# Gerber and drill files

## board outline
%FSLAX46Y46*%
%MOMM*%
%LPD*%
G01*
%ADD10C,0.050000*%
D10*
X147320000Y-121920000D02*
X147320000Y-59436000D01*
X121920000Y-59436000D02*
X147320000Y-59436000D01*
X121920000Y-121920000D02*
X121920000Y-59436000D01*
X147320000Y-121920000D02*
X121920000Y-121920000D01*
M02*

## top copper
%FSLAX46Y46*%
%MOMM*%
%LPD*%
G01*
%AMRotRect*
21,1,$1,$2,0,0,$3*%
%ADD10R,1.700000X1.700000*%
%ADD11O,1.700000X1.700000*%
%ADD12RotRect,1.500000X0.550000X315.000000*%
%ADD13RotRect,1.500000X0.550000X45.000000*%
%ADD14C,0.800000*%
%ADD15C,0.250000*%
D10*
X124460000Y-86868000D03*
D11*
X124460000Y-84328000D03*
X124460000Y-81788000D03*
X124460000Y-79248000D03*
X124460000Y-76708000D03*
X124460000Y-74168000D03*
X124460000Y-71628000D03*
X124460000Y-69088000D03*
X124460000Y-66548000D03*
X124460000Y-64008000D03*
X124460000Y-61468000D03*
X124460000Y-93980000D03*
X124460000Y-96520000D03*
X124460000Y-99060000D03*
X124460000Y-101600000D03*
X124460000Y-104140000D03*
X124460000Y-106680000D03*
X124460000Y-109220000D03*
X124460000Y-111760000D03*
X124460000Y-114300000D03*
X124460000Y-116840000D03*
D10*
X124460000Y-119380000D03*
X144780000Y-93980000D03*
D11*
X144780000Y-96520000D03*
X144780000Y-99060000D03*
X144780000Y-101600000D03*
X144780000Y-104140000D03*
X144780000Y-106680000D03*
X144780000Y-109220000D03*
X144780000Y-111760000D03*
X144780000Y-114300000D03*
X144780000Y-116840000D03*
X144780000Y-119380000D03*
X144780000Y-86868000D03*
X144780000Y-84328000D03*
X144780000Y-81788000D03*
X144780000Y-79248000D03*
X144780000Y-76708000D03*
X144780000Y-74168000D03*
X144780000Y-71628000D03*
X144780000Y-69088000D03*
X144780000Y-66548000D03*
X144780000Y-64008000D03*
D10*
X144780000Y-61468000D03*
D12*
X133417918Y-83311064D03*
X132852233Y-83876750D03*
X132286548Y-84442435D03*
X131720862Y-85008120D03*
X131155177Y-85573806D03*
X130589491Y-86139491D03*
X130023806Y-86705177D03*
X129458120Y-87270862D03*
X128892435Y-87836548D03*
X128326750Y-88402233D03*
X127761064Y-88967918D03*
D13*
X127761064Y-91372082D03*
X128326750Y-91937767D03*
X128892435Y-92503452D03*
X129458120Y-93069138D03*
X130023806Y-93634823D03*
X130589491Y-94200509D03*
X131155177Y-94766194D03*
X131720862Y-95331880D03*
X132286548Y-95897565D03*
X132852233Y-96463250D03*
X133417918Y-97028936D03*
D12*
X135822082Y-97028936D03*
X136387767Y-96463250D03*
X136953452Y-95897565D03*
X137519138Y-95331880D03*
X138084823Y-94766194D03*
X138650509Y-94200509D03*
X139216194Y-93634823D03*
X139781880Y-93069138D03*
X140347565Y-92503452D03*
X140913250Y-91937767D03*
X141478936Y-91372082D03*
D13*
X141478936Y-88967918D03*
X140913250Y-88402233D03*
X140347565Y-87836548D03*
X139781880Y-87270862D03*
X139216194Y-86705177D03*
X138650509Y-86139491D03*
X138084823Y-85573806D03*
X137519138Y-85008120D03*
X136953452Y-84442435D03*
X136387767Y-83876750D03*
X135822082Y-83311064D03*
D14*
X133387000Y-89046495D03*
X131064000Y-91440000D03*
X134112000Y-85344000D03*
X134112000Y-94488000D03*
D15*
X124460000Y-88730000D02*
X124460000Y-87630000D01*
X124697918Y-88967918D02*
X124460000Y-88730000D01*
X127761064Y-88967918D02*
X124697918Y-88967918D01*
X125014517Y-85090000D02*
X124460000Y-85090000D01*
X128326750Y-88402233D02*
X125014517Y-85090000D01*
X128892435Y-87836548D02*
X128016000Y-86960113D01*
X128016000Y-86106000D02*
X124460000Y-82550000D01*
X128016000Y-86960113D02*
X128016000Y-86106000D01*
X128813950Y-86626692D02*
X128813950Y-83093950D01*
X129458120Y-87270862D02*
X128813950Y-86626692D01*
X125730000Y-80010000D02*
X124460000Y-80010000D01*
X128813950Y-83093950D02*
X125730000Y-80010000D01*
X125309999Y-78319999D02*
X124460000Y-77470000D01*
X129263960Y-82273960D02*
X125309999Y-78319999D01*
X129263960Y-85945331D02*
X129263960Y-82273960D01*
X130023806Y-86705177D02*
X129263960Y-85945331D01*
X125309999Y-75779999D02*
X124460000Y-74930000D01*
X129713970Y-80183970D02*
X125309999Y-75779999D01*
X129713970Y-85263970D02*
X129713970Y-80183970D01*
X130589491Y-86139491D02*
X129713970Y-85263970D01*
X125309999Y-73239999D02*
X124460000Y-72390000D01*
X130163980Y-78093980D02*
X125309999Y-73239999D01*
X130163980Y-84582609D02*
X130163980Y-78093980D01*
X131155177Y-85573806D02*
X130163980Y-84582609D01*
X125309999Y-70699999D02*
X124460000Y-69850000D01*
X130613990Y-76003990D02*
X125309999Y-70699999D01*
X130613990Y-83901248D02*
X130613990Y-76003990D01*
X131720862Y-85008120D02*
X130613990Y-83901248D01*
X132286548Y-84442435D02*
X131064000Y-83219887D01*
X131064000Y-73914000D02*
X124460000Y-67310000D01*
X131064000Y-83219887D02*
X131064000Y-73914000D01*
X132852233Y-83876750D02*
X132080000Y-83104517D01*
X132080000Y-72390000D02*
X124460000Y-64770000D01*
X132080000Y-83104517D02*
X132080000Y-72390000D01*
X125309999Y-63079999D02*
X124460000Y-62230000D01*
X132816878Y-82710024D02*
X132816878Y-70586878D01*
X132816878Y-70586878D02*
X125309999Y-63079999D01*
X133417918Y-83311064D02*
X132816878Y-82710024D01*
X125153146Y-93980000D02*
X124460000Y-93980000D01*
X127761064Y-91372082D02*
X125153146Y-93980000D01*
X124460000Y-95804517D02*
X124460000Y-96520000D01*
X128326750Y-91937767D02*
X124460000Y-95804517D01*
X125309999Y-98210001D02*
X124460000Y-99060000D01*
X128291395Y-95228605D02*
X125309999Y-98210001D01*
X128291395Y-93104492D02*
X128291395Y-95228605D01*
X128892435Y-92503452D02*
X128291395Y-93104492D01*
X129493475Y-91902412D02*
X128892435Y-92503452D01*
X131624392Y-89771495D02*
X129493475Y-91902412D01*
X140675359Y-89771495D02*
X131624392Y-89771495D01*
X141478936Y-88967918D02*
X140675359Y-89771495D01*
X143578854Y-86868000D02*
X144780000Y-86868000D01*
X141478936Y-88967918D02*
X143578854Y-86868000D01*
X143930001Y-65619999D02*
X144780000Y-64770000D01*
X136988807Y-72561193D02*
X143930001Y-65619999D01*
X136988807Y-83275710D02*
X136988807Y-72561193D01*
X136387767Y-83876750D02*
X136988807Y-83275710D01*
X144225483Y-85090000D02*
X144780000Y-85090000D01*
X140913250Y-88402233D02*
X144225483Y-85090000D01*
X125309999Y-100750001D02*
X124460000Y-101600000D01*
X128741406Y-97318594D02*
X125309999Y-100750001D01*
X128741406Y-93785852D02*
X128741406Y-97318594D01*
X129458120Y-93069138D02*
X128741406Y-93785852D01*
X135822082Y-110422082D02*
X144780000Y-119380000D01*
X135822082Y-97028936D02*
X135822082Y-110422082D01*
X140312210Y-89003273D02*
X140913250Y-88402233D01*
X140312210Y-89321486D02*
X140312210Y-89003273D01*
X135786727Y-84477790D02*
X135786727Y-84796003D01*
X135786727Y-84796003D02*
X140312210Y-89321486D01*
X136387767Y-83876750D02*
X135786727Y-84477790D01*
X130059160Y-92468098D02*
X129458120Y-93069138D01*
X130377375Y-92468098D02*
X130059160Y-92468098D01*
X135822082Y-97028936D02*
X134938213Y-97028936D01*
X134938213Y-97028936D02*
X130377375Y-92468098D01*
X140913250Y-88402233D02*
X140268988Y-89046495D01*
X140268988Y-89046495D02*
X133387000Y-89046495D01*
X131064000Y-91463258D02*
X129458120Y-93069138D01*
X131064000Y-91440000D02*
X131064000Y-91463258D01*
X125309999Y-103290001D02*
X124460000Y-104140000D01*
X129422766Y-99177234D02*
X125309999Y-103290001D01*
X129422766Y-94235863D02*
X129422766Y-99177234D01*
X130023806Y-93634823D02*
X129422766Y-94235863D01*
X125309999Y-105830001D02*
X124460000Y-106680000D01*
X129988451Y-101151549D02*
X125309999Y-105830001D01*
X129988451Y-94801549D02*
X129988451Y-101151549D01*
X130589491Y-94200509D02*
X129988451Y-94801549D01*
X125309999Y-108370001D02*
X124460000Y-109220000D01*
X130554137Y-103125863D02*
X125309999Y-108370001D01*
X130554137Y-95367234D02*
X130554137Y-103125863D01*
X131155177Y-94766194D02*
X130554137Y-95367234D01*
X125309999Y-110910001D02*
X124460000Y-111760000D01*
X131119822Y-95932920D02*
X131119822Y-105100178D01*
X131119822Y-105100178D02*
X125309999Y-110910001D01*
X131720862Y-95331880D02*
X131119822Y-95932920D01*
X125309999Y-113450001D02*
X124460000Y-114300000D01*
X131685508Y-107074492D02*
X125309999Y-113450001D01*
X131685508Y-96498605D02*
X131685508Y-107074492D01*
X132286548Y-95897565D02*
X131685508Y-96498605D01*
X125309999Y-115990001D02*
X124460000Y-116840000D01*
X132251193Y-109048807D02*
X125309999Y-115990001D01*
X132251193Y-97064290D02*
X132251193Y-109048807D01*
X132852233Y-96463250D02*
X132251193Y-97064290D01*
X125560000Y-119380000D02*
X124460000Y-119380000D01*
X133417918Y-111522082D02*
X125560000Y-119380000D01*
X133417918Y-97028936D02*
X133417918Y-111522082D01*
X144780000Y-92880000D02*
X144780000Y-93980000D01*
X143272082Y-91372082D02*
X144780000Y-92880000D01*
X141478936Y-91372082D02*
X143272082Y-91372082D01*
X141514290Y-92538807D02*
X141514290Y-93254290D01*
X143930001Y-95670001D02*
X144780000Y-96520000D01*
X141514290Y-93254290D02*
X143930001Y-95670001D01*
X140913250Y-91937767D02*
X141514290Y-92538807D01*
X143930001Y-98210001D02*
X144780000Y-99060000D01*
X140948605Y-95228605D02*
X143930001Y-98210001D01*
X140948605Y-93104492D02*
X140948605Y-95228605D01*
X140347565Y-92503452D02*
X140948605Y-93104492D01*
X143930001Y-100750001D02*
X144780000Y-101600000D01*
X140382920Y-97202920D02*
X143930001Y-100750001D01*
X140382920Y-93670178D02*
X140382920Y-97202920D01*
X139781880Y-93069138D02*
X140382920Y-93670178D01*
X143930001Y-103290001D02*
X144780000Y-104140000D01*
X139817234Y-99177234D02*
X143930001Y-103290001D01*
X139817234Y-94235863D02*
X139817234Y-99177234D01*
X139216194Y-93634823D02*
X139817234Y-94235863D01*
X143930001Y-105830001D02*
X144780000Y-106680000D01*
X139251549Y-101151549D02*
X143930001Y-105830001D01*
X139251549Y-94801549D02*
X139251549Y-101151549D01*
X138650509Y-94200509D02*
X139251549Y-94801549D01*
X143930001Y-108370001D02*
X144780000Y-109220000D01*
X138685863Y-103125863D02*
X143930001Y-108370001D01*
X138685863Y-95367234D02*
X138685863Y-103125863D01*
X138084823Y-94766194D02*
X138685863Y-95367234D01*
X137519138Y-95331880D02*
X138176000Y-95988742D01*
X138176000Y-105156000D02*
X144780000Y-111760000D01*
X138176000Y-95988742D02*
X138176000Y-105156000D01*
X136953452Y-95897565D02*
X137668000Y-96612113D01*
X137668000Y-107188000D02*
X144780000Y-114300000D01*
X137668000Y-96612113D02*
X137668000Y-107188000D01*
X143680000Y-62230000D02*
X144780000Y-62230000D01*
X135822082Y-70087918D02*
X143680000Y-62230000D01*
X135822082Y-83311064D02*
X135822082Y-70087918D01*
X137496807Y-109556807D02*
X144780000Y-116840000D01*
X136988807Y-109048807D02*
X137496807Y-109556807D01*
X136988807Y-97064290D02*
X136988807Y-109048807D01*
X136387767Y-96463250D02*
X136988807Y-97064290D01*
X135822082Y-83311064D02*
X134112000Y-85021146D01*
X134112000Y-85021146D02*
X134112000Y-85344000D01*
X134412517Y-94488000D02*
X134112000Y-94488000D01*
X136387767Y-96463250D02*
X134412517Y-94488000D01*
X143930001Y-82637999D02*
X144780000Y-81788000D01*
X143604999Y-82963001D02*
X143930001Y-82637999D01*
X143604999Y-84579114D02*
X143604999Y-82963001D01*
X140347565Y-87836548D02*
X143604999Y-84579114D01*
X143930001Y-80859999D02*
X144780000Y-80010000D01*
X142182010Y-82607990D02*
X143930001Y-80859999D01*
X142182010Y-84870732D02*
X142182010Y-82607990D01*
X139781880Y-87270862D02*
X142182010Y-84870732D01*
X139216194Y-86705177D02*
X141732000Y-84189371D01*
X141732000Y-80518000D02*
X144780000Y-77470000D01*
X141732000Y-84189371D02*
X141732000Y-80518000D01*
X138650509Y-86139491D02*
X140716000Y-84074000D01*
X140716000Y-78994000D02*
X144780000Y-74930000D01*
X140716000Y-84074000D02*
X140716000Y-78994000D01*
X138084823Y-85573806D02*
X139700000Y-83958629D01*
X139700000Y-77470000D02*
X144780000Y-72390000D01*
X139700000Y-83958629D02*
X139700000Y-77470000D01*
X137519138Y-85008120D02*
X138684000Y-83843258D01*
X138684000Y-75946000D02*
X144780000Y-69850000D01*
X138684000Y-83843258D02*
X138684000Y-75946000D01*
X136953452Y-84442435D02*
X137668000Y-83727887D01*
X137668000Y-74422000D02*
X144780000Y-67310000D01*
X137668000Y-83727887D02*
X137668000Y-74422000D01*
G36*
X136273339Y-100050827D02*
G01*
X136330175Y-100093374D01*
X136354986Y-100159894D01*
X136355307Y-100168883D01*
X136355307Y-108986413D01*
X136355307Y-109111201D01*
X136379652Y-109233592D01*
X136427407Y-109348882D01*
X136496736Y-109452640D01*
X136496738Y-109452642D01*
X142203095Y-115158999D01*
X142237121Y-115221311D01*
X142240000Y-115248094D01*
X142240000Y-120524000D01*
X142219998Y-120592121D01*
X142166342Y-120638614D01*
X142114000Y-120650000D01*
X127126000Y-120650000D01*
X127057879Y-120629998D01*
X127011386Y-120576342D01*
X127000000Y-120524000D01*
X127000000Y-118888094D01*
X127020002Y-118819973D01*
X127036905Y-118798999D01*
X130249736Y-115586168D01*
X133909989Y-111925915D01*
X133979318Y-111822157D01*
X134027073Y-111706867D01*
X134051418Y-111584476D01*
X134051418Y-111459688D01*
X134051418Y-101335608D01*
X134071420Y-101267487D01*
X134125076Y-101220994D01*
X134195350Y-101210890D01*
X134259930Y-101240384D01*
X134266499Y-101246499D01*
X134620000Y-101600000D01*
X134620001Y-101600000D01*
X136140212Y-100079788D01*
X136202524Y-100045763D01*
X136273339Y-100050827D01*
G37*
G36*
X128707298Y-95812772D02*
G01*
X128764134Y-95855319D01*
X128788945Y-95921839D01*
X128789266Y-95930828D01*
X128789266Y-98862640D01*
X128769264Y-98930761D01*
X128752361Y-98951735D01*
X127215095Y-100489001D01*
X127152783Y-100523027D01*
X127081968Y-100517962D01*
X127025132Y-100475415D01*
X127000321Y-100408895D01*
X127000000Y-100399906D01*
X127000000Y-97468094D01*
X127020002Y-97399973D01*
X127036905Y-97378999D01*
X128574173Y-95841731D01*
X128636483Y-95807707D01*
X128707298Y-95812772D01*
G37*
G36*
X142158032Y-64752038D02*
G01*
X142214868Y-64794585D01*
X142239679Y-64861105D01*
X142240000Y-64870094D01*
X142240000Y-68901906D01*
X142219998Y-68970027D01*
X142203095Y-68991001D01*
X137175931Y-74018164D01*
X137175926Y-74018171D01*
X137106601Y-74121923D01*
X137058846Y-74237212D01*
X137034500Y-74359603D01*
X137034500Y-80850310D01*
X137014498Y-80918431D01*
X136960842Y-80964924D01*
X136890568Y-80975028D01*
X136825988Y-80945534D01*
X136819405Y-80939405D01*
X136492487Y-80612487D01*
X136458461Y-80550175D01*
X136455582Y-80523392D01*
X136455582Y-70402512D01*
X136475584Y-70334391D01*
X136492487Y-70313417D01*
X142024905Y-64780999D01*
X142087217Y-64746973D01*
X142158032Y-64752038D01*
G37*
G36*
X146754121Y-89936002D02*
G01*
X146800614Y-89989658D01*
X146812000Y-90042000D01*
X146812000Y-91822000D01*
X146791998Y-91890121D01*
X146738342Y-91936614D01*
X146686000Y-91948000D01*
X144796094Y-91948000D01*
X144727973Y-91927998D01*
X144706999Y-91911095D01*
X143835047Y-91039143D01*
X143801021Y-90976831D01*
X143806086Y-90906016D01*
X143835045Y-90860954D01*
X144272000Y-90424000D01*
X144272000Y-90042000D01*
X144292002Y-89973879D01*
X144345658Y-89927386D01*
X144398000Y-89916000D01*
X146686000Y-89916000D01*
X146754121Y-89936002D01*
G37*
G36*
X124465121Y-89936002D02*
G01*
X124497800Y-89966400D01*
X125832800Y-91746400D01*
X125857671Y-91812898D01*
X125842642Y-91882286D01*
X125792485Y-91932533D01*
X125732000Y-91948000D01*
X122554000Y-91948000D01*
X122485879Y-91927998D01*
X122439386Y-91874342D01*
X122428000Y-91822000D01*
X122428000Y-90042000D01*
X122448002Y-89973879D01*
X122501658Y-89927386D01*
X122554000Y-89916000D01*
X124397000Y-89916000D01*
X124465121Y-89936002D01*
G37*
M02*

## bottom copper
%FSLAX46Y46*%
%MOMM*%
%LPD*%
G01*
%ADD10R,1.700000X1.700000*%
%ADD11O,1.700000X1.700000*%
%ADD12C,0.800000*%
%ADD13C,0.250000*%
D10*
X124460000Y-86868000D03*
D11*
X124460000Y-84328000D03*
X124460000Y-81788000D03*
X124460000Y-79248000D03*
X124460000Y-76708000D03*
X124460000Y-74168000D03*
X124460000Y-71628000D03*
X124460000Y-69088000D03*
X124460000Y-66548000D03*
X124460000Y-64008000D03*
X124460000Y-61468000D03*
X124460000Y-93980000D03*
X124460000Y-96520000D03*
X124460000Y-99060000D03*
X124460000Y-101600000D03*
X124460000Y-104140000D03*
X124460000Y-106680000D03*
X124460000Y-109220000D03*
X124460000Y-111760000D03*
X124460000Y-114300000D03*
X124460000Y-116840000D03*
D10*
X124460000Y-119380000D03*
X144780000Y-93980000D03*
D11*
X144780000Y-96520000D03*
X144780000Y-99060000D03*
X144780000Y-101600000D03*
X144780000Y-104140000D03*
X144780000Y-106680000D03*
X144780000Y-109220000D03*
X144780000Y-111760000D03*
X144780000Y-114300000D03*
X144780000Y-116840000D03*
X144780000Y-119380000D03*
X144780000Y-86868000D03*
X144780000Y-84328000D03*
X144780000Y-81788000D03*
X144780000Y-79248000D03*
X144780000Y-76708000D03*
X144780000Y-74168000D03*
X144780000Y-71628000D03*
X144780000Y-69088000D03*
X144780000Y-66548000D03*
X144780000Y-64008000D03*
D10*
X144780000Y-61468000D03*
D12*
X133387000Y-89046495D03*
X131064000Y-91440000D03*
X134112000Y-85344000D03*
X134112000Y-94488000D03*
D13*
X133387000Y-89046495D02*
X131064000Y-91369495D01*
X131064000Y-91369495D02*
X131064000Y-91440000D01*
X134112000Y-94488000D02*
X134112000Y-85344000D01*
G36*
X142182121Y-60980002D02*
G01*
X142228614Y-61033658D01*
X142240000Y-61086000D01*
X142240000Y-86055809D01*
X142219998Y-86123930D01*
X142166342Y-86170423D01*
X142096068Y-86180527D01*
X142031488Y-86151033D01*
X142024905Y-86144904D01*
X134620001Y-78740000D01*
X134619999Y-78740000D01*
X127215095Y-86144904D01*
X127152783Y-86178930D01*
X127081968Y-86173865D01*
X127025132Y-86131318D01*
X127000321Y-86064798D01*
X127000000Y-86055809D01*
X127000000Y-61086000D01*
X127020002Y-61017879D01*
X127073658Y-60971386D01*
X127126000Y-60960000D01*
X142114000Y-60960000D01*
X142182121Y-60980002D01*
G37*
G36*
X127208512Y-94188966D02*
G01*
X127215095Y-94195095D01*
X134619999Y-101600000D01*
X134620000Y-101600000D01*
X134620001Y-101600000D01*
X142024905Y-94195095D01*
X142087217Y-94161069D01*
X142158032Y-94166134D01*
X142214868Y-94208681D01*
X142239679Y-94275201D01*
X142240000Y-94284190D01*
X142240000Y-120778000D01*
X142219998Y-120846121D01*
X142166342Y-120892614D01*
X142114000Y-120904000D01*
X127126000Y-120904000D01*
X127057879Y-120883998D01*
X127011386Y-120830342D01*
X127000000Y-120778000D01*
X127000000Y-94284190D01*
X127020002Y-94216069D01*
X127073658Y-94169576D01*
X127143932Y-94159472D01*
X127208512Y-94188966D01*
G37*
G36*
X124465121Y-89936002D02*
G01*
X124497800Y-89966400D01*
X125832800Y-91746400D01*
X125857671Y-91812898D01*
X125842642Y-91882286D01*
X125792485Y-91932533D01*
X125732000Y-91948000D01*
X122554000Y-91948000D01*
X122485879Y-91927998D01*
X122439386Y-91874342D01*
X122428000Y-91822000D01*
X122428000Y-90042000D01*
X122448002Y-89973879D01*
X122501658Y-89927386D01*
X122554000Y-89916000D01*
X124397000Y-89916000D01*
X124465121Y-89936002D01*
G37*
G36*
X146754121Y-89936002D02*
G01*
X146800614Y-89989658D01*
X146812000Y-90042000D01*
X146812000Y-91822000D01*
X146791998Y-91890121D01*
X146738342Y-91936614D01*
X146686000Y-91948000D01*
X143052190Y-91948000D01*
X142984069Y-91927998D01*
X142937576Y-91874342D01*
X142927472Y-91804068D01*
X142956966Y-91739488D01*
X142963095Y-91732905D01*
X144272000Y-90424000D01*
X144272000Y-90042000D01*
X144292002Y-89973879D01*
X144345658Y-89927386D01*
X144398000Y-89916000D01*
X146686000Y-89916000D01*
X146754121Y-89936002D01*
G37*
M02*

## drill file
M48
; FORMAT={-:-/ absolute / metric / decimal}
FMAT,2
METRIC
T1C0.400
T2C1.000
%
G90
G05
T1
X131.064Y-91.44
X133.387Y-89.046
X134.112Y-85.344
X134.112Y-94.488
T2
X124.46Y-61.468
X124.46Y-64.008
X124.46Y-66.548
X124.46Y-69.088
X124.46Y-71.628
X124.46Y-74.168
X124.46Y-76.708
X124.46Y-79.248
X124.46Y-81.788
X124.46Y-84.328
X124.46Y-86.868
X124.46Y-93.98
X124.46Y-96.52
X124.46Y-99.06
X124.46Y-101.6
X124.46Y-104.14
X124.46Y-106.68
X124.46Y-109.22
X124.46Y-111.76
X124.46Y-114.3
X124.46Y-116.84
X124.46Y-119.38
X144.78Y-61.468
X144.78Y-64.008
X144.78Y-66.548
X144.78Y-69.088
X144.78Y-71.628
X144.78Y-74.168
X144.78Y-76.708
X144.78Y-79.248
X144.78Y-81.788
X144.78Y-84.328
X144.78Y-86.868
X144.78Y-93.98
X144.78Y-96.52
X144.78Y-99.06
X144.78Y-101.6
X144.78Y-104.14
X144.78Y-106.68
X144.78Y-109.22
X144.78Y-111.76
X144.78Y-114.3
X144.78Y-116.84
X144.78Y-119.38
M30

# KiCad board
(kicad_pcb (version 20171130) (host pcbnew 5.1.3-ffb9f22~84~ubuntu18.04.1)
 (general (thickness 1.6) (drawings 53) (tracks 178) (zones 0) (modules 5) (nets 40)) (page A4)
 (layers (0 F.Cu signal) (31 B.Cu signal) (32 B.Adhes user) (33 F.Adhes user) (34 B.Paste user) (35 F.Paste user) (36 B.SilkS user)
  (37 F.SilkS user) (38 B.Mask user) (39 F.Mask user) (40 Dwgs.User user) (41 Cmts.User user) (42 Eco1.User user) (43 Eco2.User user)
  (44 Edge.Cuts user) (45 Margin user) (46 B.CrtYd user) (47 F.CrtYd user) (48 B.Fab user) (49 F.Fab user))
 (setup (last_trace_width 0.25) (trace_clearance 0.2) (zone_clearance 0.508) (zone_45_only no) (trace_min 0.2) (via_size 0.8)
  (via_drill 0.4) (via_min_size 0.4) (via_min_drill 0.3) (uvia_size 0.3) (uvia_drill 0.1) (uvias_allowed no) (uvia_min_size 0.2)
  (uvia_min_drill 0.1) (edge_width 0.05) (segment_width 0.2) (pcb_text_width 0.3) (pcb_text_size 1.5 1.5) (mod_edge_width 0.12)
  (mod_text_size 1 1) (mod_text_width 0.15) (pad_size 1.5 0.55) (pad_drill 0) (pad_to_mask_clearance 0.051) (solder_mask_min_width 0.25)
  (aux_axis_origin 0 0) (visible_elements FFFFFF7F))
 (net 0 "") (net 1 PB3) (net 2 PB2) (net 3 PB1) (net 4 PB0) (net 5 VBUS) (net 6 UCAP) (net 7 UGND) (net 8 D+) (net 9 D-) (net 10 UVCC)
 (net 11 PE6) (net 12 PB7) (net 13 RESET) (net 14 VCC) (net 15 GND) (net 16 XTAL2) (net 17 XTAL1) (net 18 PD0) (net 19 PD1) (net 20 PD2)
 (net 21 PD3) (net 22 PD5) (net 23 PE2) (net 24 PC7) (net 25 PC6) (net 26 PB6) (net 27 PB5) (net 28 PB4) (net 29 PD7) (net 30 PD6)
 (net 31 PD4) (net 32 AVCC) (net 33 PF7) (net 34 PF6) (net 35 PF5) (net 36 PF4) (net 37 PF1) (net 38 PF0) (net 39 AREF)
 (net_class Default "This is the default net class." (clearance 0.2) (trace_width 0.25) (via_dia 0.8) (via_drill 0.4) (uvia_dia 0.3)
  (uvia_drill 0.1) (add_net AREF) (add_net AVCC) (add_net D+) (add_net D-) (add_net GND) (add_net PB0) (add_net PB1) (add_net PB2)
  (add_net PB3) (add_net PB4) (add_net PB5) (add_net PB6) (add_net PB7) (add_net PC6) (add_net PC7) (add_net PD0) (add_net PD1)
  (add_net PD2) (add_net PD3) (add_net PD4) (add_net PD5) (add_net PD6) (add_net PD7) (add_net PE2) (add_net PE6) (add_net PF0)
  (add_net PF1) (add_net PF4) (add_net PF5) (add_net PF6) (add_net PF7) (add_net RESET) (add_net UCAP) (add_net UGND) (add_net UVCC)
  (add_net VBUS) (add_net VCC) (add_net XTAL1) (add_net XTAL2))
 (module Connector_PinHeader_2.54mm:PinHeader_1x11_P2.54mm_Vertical (layer F.Cu) (at 124.46 86.868 180)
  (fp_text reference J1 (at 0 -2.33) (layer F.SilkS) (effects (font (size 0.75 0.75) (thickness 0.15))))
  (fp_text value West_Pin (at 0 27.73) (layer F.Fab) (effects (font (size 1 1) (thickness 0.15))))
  (pad 1 thru_hole rect (at 0 0 180) (size 1.7 1.7) (drill 1) (layers *.Cu *.Mask) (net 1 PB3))
  (pad 2 thru_hole oval (at 0 2.54 180) (size 1.7 1.7) (drill 1) (layers *.Cu *.Mask) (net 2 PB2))
  (pad 3 thru_hole oval (at 0 5.08 180) (size 1.7 1.7) (drill 1) (layers *.Cu *.Mask) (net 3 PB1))
  (pad 4 thru_hole oval (at 0 7.62 180) (size 1.7 1.7) (drill 1) (layers *.Cu *.Mask) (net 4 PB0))
  (pad 5 thru_hole oval (at 0 10.16 180) (size 1.7 1.7) (drill 1) (layers *.Cu *.Mask) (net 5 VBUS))
  (pad 6 thru_hole oval (at 0 12.7 180) (size 1.7 1.7) (drill 1) (layers *.Cu *.Mask) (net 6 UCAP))
  (pad 7 thru_hole oval (at 0 15.24 180) (size 1.7 1.7) (drill 1) (layers *.Cu *.Mask) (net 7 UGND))
  (pad 8 thru_hole oval (at 0 17.78 180) (size 1.7 1.7) (drill 1) (layers *.Cu *.Mask) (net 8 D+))
  (pad 9 thru_hole oval (at 0 20.32 180) (size 1.7 1.7) (drill 1) (layers *.Cu *.Mask) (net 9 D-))
  (pad 10 thru_hole oval (at 0 22.86 180) (size 1.7 1.7) (drill 1) (layers *.Cu *.Mask) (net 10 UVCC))
  (pad 11 thru_hole oval (at 0 25.4 180) (size 1.7 1.7) (drill 1) (layers *.Cu *.Mask) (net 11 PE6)))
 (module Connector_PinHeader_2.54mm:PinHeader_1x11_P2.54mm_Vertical (layer F.Cu) (at 124.46 119.38 180)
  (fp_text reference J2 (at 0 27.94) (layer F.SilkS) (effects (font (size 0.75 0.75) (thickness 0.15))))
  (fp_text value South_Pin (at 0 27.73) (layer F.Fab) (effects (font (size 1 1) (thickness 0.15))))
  (pad 11 thru_hole oval (at 0 25.4 180) (size 1.7 1.7) (drill 1) (layers *.Cu *.Mask) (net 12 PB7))
  (pad 10 thru_hole oval (at 0 22.86 180) (size 1.7 1.7) (drill 1) (layers *.Cu *.Mask) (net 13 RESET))
  (pad 9 thru_hole oval (at 0 20.32 180) (size 1.7 1.7) (drill 1) (layers *.Cu *.Mask) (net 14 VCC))
  (pad 8 thru_hole oval (at 0 17.78 180) (size 1.7 1.7) (drill 1) (layers *.Cu *.Mask) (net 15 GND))
  (pad 7 thru_hole oval (at 0 15.24 180) (size 1.7 1.7) (drill 1) (layers *.Cu *.Mask) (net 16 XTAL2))
  (pad 6 thru_hole oval (at 0 12.7 180) (size 1.7 1.7) (drill 1) (layers *.Cu *.Mask) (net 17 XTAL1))
  (pad 5 thru_hole oval (at 0 10.16 180) (size 1.7 1.7) (drill 1) (layers *.Cu *.Mask) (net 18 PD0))
  (pad 4 thru_hole oval (at 0 7.62 180) (size 1.7 1.7) (drill 1) (layers *.Cu *.Mask) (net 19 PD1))
  (pad 3 thru_hole oval (at 0 5.08 180) (size 1.7 1.7) (drill 1) (layers *.Cu *.Mask) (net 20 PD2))
  (pad 2 thru_hole oval (at 0 2.54 180) (size 1.7 1.7) (drill 1) (layers *.Cu *.Mask) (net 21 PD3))
  (pad 1 thru_hole rect (at 0 0 180) (size 1.7 1.7) (drill 1) (layers *.Cu *.Mask) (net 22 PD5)))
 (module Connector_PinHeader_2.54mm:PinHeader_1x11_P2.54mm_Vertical (layer F.Cu) (at 144.78 93.98)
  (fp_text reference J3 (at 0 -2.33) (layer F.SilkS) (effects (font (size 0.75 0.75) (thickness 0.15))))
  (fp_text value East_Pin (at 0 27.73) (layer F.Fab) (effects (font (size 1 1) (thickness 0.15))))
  (pad 1 thru_hole rect (at 0 0) (size 1.7 1.7) (drill 1) (layers *.Cu *.Mask) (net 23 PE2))
  (pad 2 thru_hole oval (at 0 2.54) (size 1.7 1.7) (drill 1) (layers *.Cu *.Mask) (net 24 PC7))
  (pad 3 thru_hole oval (at 0 5.08) (size 1.7 1.7) (drill 1) (layers *.Cu *.Mask) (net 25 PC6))
  (pad 4 thru_hole oval (at 0 7.62) (size 1.7 1.7) (drill 1) (layers *.Cu *.Mask) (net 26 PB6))
  (pad 5 thru_hole oval (at 0 10.16) (size 1.7 1.7) (drill 1) (layers *.Cu *.Mask) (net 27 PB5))
  (pad 6 thru_hole oval (at 0 12.7) (size 1.7 1.7) (drill 1) (layers *.Cu *.Mask) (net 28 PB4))
  (pad 7 thru_hole oval (at 0 15.24) (size 1.7 1.7) (drill 1) (layers *.Cu *.Mask) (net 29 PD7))
  (pad 8 thru_hole oval (at 0 17.78) (size 1.7 1.7) (drill 1) (layers *.Cu *.Mask) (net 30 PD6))
  (pad 9 thru_hole oval (at 0 20.32) (size 1.7 1.7) (drill 1) (layers *.Cu *.Mask) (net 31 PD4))
  (pad 10 thru_hole oval (at 0 22.86) (size 1.7 1.7) (drill 1) (layers *.Cu *.Mask) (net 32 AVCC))
  (pad 11 thru_hole oval (at 0 25.4) (size 1.7 1.7) (drill 1) (layers *.Cu *.Mask) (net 15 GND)))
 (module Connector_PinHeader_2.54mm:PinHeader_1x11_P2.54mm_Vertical (layer F.Cu) (at 144.78 61.468)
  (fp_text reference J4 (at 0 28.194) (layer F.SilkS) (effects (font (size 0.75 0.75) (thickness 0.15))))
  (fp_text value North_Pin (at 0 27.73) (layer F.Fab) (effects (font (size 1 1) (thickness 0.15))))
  (pad 11 thru_hole oval (at 0 25.4) (size 1.7 1.7) (drill 1) (layers *.Cu *.Mask) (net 14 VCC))
  (pad 10 thru_hole oval (at 0 22.86) (size 1.7 1.7) (drill 1) (layers *.Cu *.Mask) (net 15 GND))
  (pad 9 thru_hole oval (at 0 20.32) (size 1.7 1.7) (drill 1) (layers *.Cu *.Mask) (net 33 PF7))
  (pad 8 thru_hole oval (at 0 17.78) (size 1.7 1.7) (drill 1) (layers *.Cu *.Mask) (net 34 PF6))
  (pad 7 thru_hole oval (at 0 15.24) (size 1.7 1.7) (drill 1) (layers *.Cu *.Mask) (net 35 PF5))
  (pad 6 thru_hole oval (at 0 12.7) (size 1.7 1.7) (drill 1) (layers *.Cu *.Mask) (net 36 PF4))
  (pad 5 thru_hole oval (at 0 10.16) (size 1.7 1.7) (drill 1) (layers *.Cu *.Mask) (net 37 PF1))
  (pad 4 thru_hole oval (at 0 7.62) (size 1.7 1.7) (drill 1) (layers *.Cu *.Mask) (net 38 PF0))
  (pad 3 thru_hole oval (at 0 5.08) (size 1.7 1.7) (drill 1) (layers *.Cu *.Mask) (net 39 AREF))
  (pad 2 thru_hole oval (at 0 2.54) (size 1.7 1.7) (drill 1) (layers *.Cu *.Mask) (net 15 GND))
  (pad 1 thru_hole rect (at 0 0) (size 1.7 1.7) (drill 1) (layers *.Cu *.Mask) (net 32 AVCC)))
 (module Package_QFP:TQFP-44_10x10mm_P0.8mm (layer F.Cu) (at 134.62 90.17 315)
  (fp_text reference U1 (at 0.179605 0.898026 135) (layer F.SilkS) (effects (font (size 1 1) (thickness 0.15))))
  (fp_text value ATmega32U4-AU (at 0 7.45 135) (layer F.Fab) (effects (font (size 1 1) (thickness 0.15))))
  (pad 1 smd rect (at -5.7 -4 315) (size 1.5 0.55) (layers F.Cu F.Paste F.Mask) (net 11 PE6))
  (pad 2 smd rect (at -5.7 -3.2 315) (size 1.5 0.55) (layers F.Cu F.Paste F.Mask) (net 10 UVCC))
  (pad 3 smd rect (at -5.7 -2.4 315) (size 1.5 0.55) (layers F.Cu F.Paste F.Mask) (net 9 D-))
  (pad 4 smd rect (at -5.7 -1.6 315) (size 1.5 0.55) (layers F.Cu F.Paste F.Mask) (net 8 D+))
  (pad 5 smd rect (at -5.7 -0.8 315) (size 1.5 0.55) (layers F.Cu F.Paste F.Mask) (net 7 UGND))
  (pad 6 smd rect (at -5.7 0 315) (size 1.5 0.55) (layers F.Cu F.Paste F.Mask) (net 6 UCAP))
  (pad 7 smd rect (at -5.7 0.8 315) (size 1.5 0.55) (layers F.Cu F.Paste F.Mask) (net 5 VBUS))
  (pad 8 smd rect (at -5.7 1.6 315) (size 1.5 0.55) (layers F.Cu F.Paste F.Mask) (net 4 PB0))
  (pad 9 smd rect (at -5.7 2.4 315) (size 1.5 0.55) (layers F.Cu F.Paste F.Mask) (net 3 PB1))
  (pad 10 smd rect (at -5.7 3.2 315) (size 1.5 0.55) (layers F.Cu F.Paste F.Mask) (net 2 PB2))
  (pad 11 smd rect (at -5.7 4 315) (size 1.5 0.55) (layers F.Cu F.Paste F.Mask) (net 1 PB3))
  (pad 12 smd rect (at -4 5.7 45) (size 1.5 0.55) (layers F.Cu F.Paste F.Mask) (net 12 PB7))
  (pad 13 smd rect (at -3.2 5.7 45) (size 1.5 0.55) (layers F.Cu F.Paste F.Mask) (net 13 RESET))
  (pad 14 smd rect (at -2.4 5.7 45) (size 1.5 0.55) (layers F.Cu F.Paste F.Mask) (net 14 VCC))
  (pad 15 smd rect (at -1.6 5.7 45) (size 1.5 0.55) (layers F.Cu F.Paste F.Mask) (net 15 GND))
  (pad 16 smd rect (at -0.8 5.7 45) (size 1.5 0.55) (layers F.Cu F.Paste F.Mask) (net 16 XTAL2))
  (pad 17 smd rect (at 0 5.7 45) (size 1.5 0.55) (layers F.Cu F.Paste F.Mask) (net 17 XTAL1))
  (pad 18 smd rect (at 0.8 5.7 45) (size 1.5 0.55) (layers F.Cu F.Paste F.Mask) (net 18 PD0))
  (pad 19 smd rect (at 1.6 5.7 45) (size 1.5 0.55) (layers F.Cu F.Paste F.Mask) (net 19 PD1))
  (pad 20 smd rect (at 2.4 5.7 45) (size 1.5 0.55) (layers F.Cu F.Paste F.Mask) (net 20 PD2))
  (pad 21 smd rect (at 3.2 5.7 45) (size 1.5 0.55) (layers F.Cu F.Paste F.Mask) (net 21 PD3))
  (pad 22 smd rect (at 4 5.7 45) (size 1.5 0.55) (layers F.Cu F.Paste F.Mask) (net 22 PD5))
  (pad 23 smd rect (at 5.7 4 315) (size 1.5 0.55) (layers F.Cu F.Paste F.Mask) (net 15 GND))
  (pad 24 smd rect (at 5.7 3.2 315) (size 1.5 0.55) (layers F.Cu F.Paste F.Mask) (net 32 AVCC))
  (pad 25 smd rect (at 5.7 2.4 315) (size 1.5 0.55) (layers F.Cu F.Paste F.Mask) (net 31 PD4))
  (pad 26 smd rect (at 5.7 1.6 315) (size 1.5 0.55) (layers F.Cu F.Paste F.Mask) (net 30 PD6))
  (pad 27 smd rect (at 5.7 0.8 315) (size 1.5 0.55) (layers F.Cu F.Paste F.Mask) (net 29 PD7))
  (pad 28 smd rect (at 5.7 0 315) (size 1.5 0.55) (layers F.Cu F.Paste F.Mask) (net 28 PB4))
  (pad 29 smd rect (at 5.7 -0.8 315) (size 1.5 0.55) (layers F.Cu F.Paste F.Mask) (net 27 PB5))
  (pad 30 smd rect (at 5.7 -1.6 315) (size 1.5 0.55) (layers F.Cu F.Paste F.Mask) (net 26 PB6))
  (pad 31 smd rect (at 5.7 -2.4 315) (size 1.5 0.55) (layers F.Cu F.Paste F.Mask) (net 25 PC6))
  (pad 32 smd rect (at 5.7 -3.2 315) (size 1.5 0.55) (layers F.Cu F.Paste F.Mask) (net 24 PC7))
  (pad 33 smd rect (at 5.7 -4 315) (size 1.5 0.55) (layers F.Cu F.Paste F.Mask) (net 23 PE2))
  (pad 34 smd rect (at 4 -5.7 45) (size 1.5 0.55) (layers F.Cu F.Paste F.Mask) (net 14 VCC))
  (pad 35 smd rect (at 3.2 -5.7 45) (size 1.5 0.55) (layers F.Cu F.Paste F.Mask) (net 15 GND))
  (pad 36 smd rect (at 2.4 -5.7 45) (size 1.5 0.55) (layers F.Cu F.Paste F.Mask) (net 33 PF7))
  (pad 37 smd rect (at 1.6 -5.7 45) (size 1.5 0.55) (layers F.Cu F.Paste F.Mask) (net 34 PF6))
  (pad 38 smd rect (at 0.8 -5.7 45) (size 1.5 0.55) (layers F.Cu F.Paste F.Mask) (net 35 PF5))
  (pad 39 smd rect (at 0 -5.7 45) (size 1.5 0.55) (layers F.Cu F.Paste F.Mask) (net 36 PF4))
  (pad 40 smd rect (at -0.8 -5.7 45) (size 1.5 0.55) (layers F.Cu F.Paste F.Mask) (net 37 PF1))
  (pad 41 smd rect (at -1.6 -5.7 45) (size 1.5 0.55) (layers F.Cu F.Paste F.Mask) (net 38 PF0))
  (pad 42 smd rect (at -2.4 -5.7 45) (size 1.5 0.55) (layers F.Cu F.Paste F.Mask) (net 39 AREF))
  (pad 43 smd rect (at -3.2 -5.7 45) (size 1.5 0.55) (layers F.Cu F.Paste F.Mask) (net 15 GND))
  (pad 44 smd rect (at -4 -5.7 45) (size 1.5 0.55) (layers F.Cu F.Paste F.Mask) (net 32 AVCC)))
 (gr_line (start 147.32 121.92) (end 147.32 59.436) (layer Edge.Cuts) (width 0.05))
 (gr_line (start 121.92 59.436) (end 147.32 59.436) (layer Edge.Cuts) (width 0.05))
 (gr_line (start 121.92 121.92) (end 121.92 59.436) (layer Edge.Cuts) (width 0.05))
 (gr_line (start 147.32 121.92) (end 121.92 121.92) (layer Edge.Cuts) (width 0.05))
 (segment (start 124.46 88.73) (end 124.46 87.63) (width 0.25) (layer F.Cu) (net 1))
 (segment (start 124.697918 88.967918) (end 124.46 88.73) (width 0.25) (layer F.Cu) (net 1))
 (segment (start 127.761064 88.967918) (end 124.697918 88.967918) (width 0.25) (layer F.Cu) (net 1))
 (segment (start 125.014517 85.09) (end 124.46 85.09) (width 0.25) (layer F.Cu) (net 2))
 (segment (start 128.32675 88.402233) (end 125.014517 85.09) (width 0.25) (layer F.Cu) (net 2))
 (segment (start 128.892435 87.836548) (end 128.016 86.960113) (width 0.25) (layer F.Cu) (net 3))
 (segment (start 128.016 86.106) (end 124.46 82.55) (width 0.25) (layer F.Cu) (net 3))
 (segment (start 128.016 86.960113) (end 128.016 86.106) (width 0.25) (layer F.Cu) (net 3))
 (segment (start 128.81395 86.626692) (end 128.81395 83.09395) (width 0.25) (layer F.Cu) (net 4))
 (segment (start 129.45812 87.270862) (end 128.81395 86.626692) (width 0.25) (layer F.Cu) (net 4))
 (segment (start 125.73 80.01) (end 124.46 80.01) (width 0.25) (layer F.Cu) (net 4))
 (segment (start 128.81395 83.09395) (end 125.73 80.01) (width 0.25) (layer F.Cu) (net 4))
 (segment (start 125.309999 78.319999) (end 124.46 77.47) (width 0.25) (layer F.Cu) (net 5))
 (segment (start 129.26396 82.27396) (end 125.309999 78.319999) (width 0.25) (layer F.Cu) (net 5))
 (segment (start 129.26396 85.945331) (end 129.26396 82.27396) (width 0.25) (layer F.Cu) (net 5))
 (segment (start 130.023806 86.705177) (end 129.26396 85.945331) (width 0.25) (layer F.Cu) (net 5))
 (segment (start 125.309999 75.779999) (end 124.46 74.93) (width 0.25) (layer F.Cu) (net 6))
 (segment (start 129.71397 80.18397) (end 125.309999 75.779999) (width 0.25) (layer F.Cu) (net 6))
 (segment (start 129.71397 85.26397) (end 129.71397 80.18397) (width 0.25) (layer F.Cu) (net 6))
 (segment (start 130.589491 86.139491) (end 129.71397 85.26397) (width 0.25) (layer F.Cu) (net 6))
 (segment (start 125.309999 73.239999) (end 124.46 72.39) (width 0.25) (layer F.Cu) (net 7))
 (segment (start 130.16398 78.09398) (end 125.309999 73.239999) (width 0.25) (layer F.Cu) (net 7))
 (segment (start 130.16398 84.582609) (end 130.16398 78.09398) (width 0.25) (layer F.Cu) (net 7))
 (segment (start 131.155177 85.573806) (end 130.16398 84.582609) (width 0.25) (layer F.Cu) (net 7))
 (segment (start 125.309999 70.699999) (end 124.46 69.85) (width 0.25) (layer F.Cu) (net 8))
 (segment (start 130.61399 76.00399) (end 125.309999 70.699999) (width 0.25) (layer F.Cu) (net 8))
 (segment (start 130.61399 83.901248) (end 130.61399 76.00399) (width 0.25) (layer F.Cu) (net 8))
 (segment (start 131.720862 85.00812) (end 130.61399 83.901248) (width 0.25) (layer F.Cu) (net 8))
 (segment (start 132.286548 84.442435) (end 131.064 83.219887) (width 0.25) (layer F.Cu) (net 9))
 (segment (start 131.064 73.914) (end 124.46 67.31) (width 0.25) (layer F.Cu) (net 9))
 (segment (start 131.064 83.219887) (end 131.064 73.914) (width 0.25) (layer F.Cu) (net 9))
 (segment (start 132.852233 83.87675) (end 132.08 83.104517) (width 0.25) (layer F.Cu) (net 10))
 (segment (start 132.08 72.39) (end 124.46 64.77) (width 0.25) (layer F.Cu) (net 10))
 (segment (start 132.08 83.104517) (end 132.08 72.39) (width 0.25) (layer F.Cu) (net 10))
 (segment (start 125.309999 63.079999) (end 124.46 62.23) (width 0.25) (layer F.Cu) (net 11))
 (segment (start 132.816878 82.710024) (end 132.816878 70.586878) (width 0.25) (layer F.Cu) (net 11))
 (segment (start 132.816878 70.586878) (end 125.309999 63.079999) (width 0.25) (layer F.Cu) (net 11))
 (segment (start 133.417918 83.311064) (end 132.816878 82.710024) (width 0.25) (layer F.Cu) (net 11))
 (segment (start 125.153146 93.98) (end 124.46 93.98) (width 0.25) (layer F.Cu) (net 12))
 (segment (start 127.761064 91.372082) (end 125.153146 93.98) (width 0.25) (layer F.Cu) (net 12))
 (segment (start 124.46 95.804517) (end 124.46 96.52) (width 0.25) (layer F.Cu) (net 13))
 (segment (start 128.32675 91.937767) (end 124.46 95.804517) (width 0.25) (layer F.Cu) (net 13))
 (segment (start 125.309999 98.210001) (end 124.46 99.06) (width 0.25) (layer F.Cu) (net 14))
 (segment (start 128.291395 95.228605) (end 125.309999 98.210001) (width 0.25) (layer F.Cu) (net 14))
 (segment (start 128.291395 93.104492) (end 128.291395 95.228605) (width 0.25) (layer F.Cu) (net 14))
 (segment (start 128.892435 92.503452) (end 128.291395 93.104492) (width 0.25) (layer F.Cu) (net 14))
 (segment (start 129.493475 91.902412) (end 128.892435 92.503452) (width 0.25) (layer F.Cu) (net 14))
 (segment (start 131.624392 89.771495) (end 129.493475 91.902412) (width 0.25) (layer F.Cu) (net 14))
 (segment (start 140.675359 89.771495) (end 131.624392 89.771495) (width 0.25) (layer F.Cu) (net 14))
 (segment (start 141.478936 88.967918) (end 140.675359 89.771495) (width 0.25) (layer F.Cu) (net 14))
 (segment (start 143.578854 86.868) (end 144.78 86.868) (width 0.25) (layer F.Cu) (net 14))
 (segment (start 141.478936 88.967918) (end 143.578854 86.868) (width 0.25) (layer F.Cu) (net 14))
 (segment (start 143.930001 65.619999) (end 144.78 64.77) (width 0.25) (layer F.Cu) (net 15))
 (segment (start 136.988807 72.561193) (end 143.930001 65.619999) (width 0.25) (layer F.Cu) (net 15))
 (segment (start 136.988807 83.27571) (end 136.988807 72.561193) (width 0.25) (layer F.Cu) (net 15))
 (segment (start 136.387767 83.87675) (end 136.988807 83.27571) (width 0.25) (layer F.Cu) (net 15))
 (segment (start 144.225483 85.09) (end 144.78 85.09) (width 0.25) (layer F.Cu) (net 15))
 (segment (start 140.91325 88.402233) (end 144.225483 85.09) (width 0.25) (layer F.Cu) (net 15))
 (segment (start 125.309999 100.750001) (end 124.46 101.6) (width 0.25) (layer F.Cu) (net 15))
 (segment (start 128.741406 97.318594) (end 125.309999 100.750001) (width 0.25) (layer F.Cu) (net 15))
 (segment (start 128.741406 93.785852) (end 128.741406 97.318594) (width 0.25) (layer F.Cu) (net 15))
 (segment (start 129.45812 93.069138) (end 128.741406 93.785852) (width 0.25) (layer F.Cu) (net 15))
 (segment (start 135.822082 110.422082) (end 144.78 119.38) (width 0.25) (layer F.Cu) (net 15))
 (segment (start 135.822082 97.028936) (end 135.822082 110.422082) (width 0.25) (layer F.Cu) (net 15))
 (segment (start 140.31221 89.003273) (end 140.91325 88.402233) (width 0.25) (layer F.Cu) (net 15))
 (segment (start 140.31221 89.321486) (end 140.31221 89.003273) (width 0.25) (layer F.Cu) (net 15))
 (segment (start 135.786727 84.47779) (end 135.786727 84.796003) (width 0.25) (layer F.Cu) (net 15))
 (segment (start 135.786727 84.796003) (end 140.31221 89.321486) (width 0.25) (layer F.Cu) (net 15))
 (segment (start 136.387767 83.87675) (end 135.786727 84.47779) (width 0.25) (layer F.Cu) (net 15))
 (segment (start 130.05916 92.468098) (end 129.45812 93.069138) (width 0.25) (layer F.Cu) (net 15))
 (segment (start 130.377375 92.468098) (end 130.05916 92.468098) (width 0.25) (layer F.Cu) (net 15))
 (segment (start 135.822082 97.028936) (end 134.938213 97.028936) (width 0.25) (layer F.Cu) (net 15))
 (segment (start 134.938213 97.028936) (end 130.377375 92.468098) (width 0.25) (layer F.Cu) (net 15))
 (via (at 133.387 89.046495) (size 0.8) (drill 0.4) (layers F.Cu B.Cu) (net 15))
 (segment (start 140.91325 88.402233) (end 140.268988 89.046495) (width 0.25) (layer F.Cu) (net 15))
 (segment (start 140.268988 89.046495) (end 133.387 89.046495) (width 0.25) (layer F.Cu) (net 15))
 (segment (start 133.387 89.046495) (end 131.064 91.369495) (width 0.25) (layer B.Cu) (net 15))
 (via (at 131.064 91.44) (size 0.8) (drill 0.4) (layers F.Cu B.Cu) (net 15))
 (segment (start 131.064 91.369495) (end 131.064 91.44) (width 0.25) (layer B.Cu) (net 15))
 (segment (start 131.064 91.463258) (end 129.45812 93.069138) (width 0.25) (layer F.Cu) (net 15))
 (segment (start 131.064 91.44) (end 131.064 91.463258) (width 0.25) (layer F.Cu) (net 15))
 (segment (start 125.309999 103.290001) (end 124.46 104.14) (width 0.25) (layer F.Cu) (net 16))
 (segment (start 129.422766 99.177234) (end 125.309999 103.290001) (width 0.25) (layer F.Cu) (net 16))
 (segment (start 129.422766 94.235863) (end 129.422766 99.177234) (width 0.25) (layer F.Cu) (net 16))
 (segment (start 130.023806 93.634823) (end 129.422766 94.235863) (width 0.25) (layer F.Cu) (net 16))
 (segment (start 125.309999 105.830001) (end 124.46 106.68) (width 0.25) (layer F.Cu) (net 17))
 (segment (start 129.988451 101.151549) (end 125.309999 105.830001) (width 0.25) (layer F.Cu) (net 17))
 (segment (start 129.988451 94.801549) (end 129.988451 101.151549) (width 0.25) (layer F.Cu) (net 17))
 (segment (start 130.589491 94.200509) (end 129.988451 94.801549) (width 0.25) (layer F.Cu) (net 17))
 (segment (start 125.309999 108.370001) (end 124.46 109.22) (width 0.25) (layer F.Cu) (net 18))
 (segment (start 130.554137 103.125863) (end 125.309999 108.370001) (width 0.25) (layer F.Cu) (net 18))
 (segment (start 130.554137 95.367234) (end 130.554137 103.125863) (width 0.25) (layer F.Cu) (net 18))
 (segment (start 131.155177 94.766194) (end 130.554137 95.367234) (width 0.25) (layer F.Cu) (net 18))
 (segment (start 125.309999 110.910001) (end 124.46 111.76) (width 0.25) (layer F.Cu) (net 19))
 (segment (start 131.119822 95.93292) (end 131.119822 105.100178) (width 0.25) (layer F.Cu) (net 19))
 (segment (start 131.119822 105.100178) (end 125.309999 110.910001) (width 0.25) (layer F.Cu) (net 19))
 (segment (start 131.720862 95.33188) (end 131.119822 95.93292) (width 0.25) (layer F.Cu) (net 19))
 (segment (start 125.309999 113.450001) (end 124.46 114.3) (width 0.25) (layer F.Cu) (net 20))
 (segment (start 131.685508 107.074492) (end 125.309999 113.450001) (width 0.25) (layer F.Cu) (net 20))
 (segment (start 131.685508 96.498605) (end 131.685508 107.074492) (width 0.25) (layer F.Cu) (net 20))
 (segment (start 132.286548 95.897565) (end 131.685508 96.498605) (width 0.25) (layer F.Cu) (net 20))
 (segment (start 125.309999 115.990001) (end 124.46 116.84) (width 0.25) (layer F.Cu) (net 21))
 (segment (start 132.251193 109.048807) (end 125.309999 115.990001) (width 0.25) (layer F.Cu) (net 21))
 (segment (start 132.251193 97.06429) (end 132.251193 109.048807) (width 0.25) (layer F.Cu) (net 21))
 (segment (start 132.852233 96.46325) (end 132.251193 97.06429) (width 0.25) (layer F.Cu) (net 21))
 (segment (start 125.56 119.38) (end 124.46 119.38) (width 0.25) (layer F.Cu) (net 22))
 (segment (start 133.417918 111.522082) (end 125.56 119.38) (width 0.25) (layer F.Cu) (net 22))
 (segment (start 133.417918 97.028936) (end 133.417918 111.522082) (width 0.25) (layer F.Cu) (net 22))
 (segment (start 144.78 92.88) (end 144.78 93.98) (width 0.25) (layer F.Cu) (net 23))
 (segment (start 143.272082 91.372082) (end 144.78 92.88) (width 0.25) (layer F.Cu) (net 23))
 (segment (start 141.478936 91.372082) (end 143.272082 91.372082) (width 0.25) (layer F.Cu) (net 23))
 (segment (start 141.51429 92.538807) (end 141.51429 93.25429) (width 0.25) (layer F.Cu) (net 24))
 (segment (start 143.930001 95.670001) (end 144.78 96.52) (width 0.25) (layer F.Cu) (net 24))
 (segment (start 141.51429 93.25429) (end 143.930001 95.670001) (width 0.25) (layer F.Cu) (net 24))
 (segment (start 140.91325 91.937767) (end 141.51429 92.538807) (width 0.25) (layer F.Cu) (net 24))
 (segment (start 143.930001 98.210001) (end 144.78 99.06) (width 0.25) (layer F.Cu) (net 25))
 (segment (start 140.948605 95.228605) (end 143.930001 98.210001) (width 0.25) (layer F.Cu) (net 25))
 (segment (start 140.948605 93.104492) (end 140.948605 95.228605) (width 0.25) (layer F.Cu) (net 25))
 (segment (start 140.347565 92.503452) (end 140.948605 93.104492) (width 0.25) (layer F.Cu) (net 25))
 (segment (start 143.930001 100.750001) (end 144.78 101.6) (width 0.25) (layer F.Cu) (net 26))
 (segment (start 140.38292 97.20292) (end 143.930001 100.750001) (width 0.25) (layer F.Cu) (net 26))
 (segment (start 140.38292 93.670178) (end 140.38292 97.20292) (width 0.25) (layer F.Cu) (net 26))
 (segment (start 139.78188 93.069138) (end 140.38292 93.670178) (width 0.25) (layer F.Cu) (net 26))
 (segment (start 143.930001 103.290001) (end 144.78 104.14) (width 0.25) (layer F.Cu) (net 27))
 (segment (start 139.817234 99.177234) (end 143.930001 103.290001) (width 0.25) (layer F.Cu) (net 27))
 (segment (start 139.817234 94.235863) (end 139.817234 99.177234) (width 0.25) (layer F.Cu) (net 27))
 (segment (start 139.216194 93.634823) (end 139.817234 94.235863) (width 0.25) (layer F.Cu) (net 27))
 (segment (start 143.930001 105.830001) (end 144.78 106.68) (width 0.25) (layer F.Cu) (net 28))
 (segment (start 139.251549 101.151549) (end 143.930001 105.830001) (width 0.25) (layer F.Cu) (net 28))
 (segment (start 139.251549 94.801549) (end 139.251549 101.151549) (width 0.25) (layer F.Cu) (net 28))
 (segment (start 138.650509 94.200509) (end 139.251549 94.801549) (width 0.25) (layer F.Cu) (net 28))
 (segment (start 143.930001 108.370001) (end 144.78 109.22) (width 0.25) (layer F.Cu) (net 29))
 (segment (start 138.685863 103.125863) (end 143.930001 108.370001) (width 0.25) (layer F.Cu) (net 29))
 (segment (start 138.685863 95.367234) (end 138.685863 103.125863) (width 0.25) (layer F.Cu) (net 29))
 (segment (start 138.084823 94.766194) (end 138.685863 95.367234) (width 0.25) (layer F.Cu) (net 29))
 (segment (start 137.519138 95.33188) (end 138.176 95.988742) (width 0.25) (layer F.Cu) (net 30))
 (segment (start 138.176 105.156) (end 144.78 111.76) (width 0.25) (layer F.Cu) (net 30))
 (segment (start 138.176 95.988742) (end 138.176 105.156) (width 0.25) (layer F.Cu) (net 30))
 (segment (start 136.953452 95.897565) (end 137.668 96.612113) (width 0.25) (layer F.Cu) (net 31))
 (segment (start 137.668 107.188) (end 144.78 114.3) (width 0.25) (layer F.Cu) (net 31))
 (segment (start 137.668 96.612113) (end 137.668 107.188) (width 0.25) (layer F.Cu) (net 31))
 (segment (start 143.68 62.23) (end 144.78 62.23) (width 0.25) (layer F.Cu) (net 32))
 (segment (start 135.822082 70.087918) (end 143.68 62.23) (width 0.25) (layer F.Cu) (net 32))
 (segment (start 135.822082 83.311064) (end 135.822082 70.087918) (width 0.25) (layer F.Cu) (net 32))
 (segment (start 137.496807 109.556807) (end 144.78 116.84) (width 0.25) (layer F.Cu) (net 32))
 (segment (start 136.988807 109.048807) (end 137.496807 109.556807) (width 0.25) (layer F.Cu) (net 32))
 (segment (start 136.988807 97.06429) (end 136.988807 109.048807) (width 0.25) (layer F.Cu) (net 32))
 (segment (start 136.387767 96.46325) (end 136.988807 97.06429) (width 0.25) (layer F.Cu) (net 32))
 (via (at 134.112 85.344) (size 0.8) (drill 0.4) (layers F.Cu B.Cu) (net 32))
 (segment (start 135.822082 83.311064) (end 134.112 85.021146) (width 0.25) (layer F.Cu) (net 32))
 (segment (start 134.112 85.021146) (end 134.112 85.344) (width 0.25) (layer F.Cu) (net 32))
 (segment (start 134.112 94.488) (end 134.112 85.344) (width 0.25) (layer B.Cu) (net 32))
 (via (at 134.112 94.488) (size 0.8) (drill 0.4) (layers F.Cu B.Cu) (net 32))
 (segment (start 134.412517 94.488) (end 134.112 94.488) (width 0.25) (layer F.Cu) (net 32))
 (segment (start 136.387767 96.46325) (end 134.412517 94.488) (width 0.25) (layer F.Cu) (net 32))
 (segment (start 143.930001 82.637999) (end 144.78 81.788) (width 0.25) (layer F.Cu) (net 33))
 (segment (start 143.604999 82.963001) (end 143.930001 82.637999) (width 0.25) (layer F.Cu) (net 33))
 (segment (start 143.604999 84.579114) (end 143.604999 82.963001) (width 0.25) (layer F.Cu) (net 33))
 (segment (start 140.347565 87.836548) (end 143.604999 84.579114) (width 0.25) (layer F.Cu) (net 33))
 (segment (start 143.930001 80.859999) (end 144.78 80.01) (width 0.25) (layer F.Cu) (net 34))
 (segment (start 142.18201 82.60799) (end 143.930001 80.859999) (width 0.25) (layer F.Cu) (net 34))
 (segment (start 142.18201 84.870732) (end 142.18201 82.60799) (width 0.25) (layer F.Cu) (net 34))
 (segment (start 139.78188 87.270862) (end 142.18201 84.870732) (width 0.25) (layer F.Cu) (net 34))
 (segment (start 139.216194 86.705177) (end 141.732 84.189371) (width 0.25) (layer F.Cu) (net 35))
 (segment (start 141.732 80.518) (end 144.78 77.47) (width 0.25) (layer F.Cu) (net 35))
 (segment (start 141.732 84.189371) (end 141.732 80.518) (width 0.25) (layer F.Cu) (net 35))
 (segment (start 138.650509 86.139491) (end 140.716 84.074) (width 0.25) (layer F.Cu) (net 36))
 (segment (start 140.716 78.994) (end 144.78 74.93) (width 0.25) (layer F.Cu) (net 36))
 (segment (start 140.716 84.074) (end 140.716 78.994) (width 0.25) (layer F.Cu) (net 36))
 (segment (start 138.084823 85.573806) (end 139.7 83.958629) (width 0.25) (layer F.Cu) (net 37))
 (segment (start 139.7 77.47) (end 144.78 72.39) (width 0.25) (layer F.Cu) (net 37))
 (segment (start 139.7 83.958629) (end 139.7 77.47) (width 0.25) (layer F.Cu) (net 37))
 (segment (start 137.519138 85.00812) (end 138.684 83.843258) (width 0.25) (layer F.Cu) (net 38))
 (segment (start 138.684 75.946) (end 144.78 69.85) (width 0.25) (layer F.Cu) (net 38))
 (segment (start 138.684 83.843258) (end 138.684 75.946) (width 0.25) (layer F.Cu) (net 38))
 (segment (start 136.953452 84.442435) (end 137.668 83.727887) (width 0.25) (layer F.Cu) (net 39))
 (segment (start 137.668 74.422) (end 144.78 67.31) (width 0.25) (layer F.Cu) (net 39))
 (segment (start 137.668 83.727887) (end 137.668 74.422) (width 0.25) (layer F.Cu) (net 39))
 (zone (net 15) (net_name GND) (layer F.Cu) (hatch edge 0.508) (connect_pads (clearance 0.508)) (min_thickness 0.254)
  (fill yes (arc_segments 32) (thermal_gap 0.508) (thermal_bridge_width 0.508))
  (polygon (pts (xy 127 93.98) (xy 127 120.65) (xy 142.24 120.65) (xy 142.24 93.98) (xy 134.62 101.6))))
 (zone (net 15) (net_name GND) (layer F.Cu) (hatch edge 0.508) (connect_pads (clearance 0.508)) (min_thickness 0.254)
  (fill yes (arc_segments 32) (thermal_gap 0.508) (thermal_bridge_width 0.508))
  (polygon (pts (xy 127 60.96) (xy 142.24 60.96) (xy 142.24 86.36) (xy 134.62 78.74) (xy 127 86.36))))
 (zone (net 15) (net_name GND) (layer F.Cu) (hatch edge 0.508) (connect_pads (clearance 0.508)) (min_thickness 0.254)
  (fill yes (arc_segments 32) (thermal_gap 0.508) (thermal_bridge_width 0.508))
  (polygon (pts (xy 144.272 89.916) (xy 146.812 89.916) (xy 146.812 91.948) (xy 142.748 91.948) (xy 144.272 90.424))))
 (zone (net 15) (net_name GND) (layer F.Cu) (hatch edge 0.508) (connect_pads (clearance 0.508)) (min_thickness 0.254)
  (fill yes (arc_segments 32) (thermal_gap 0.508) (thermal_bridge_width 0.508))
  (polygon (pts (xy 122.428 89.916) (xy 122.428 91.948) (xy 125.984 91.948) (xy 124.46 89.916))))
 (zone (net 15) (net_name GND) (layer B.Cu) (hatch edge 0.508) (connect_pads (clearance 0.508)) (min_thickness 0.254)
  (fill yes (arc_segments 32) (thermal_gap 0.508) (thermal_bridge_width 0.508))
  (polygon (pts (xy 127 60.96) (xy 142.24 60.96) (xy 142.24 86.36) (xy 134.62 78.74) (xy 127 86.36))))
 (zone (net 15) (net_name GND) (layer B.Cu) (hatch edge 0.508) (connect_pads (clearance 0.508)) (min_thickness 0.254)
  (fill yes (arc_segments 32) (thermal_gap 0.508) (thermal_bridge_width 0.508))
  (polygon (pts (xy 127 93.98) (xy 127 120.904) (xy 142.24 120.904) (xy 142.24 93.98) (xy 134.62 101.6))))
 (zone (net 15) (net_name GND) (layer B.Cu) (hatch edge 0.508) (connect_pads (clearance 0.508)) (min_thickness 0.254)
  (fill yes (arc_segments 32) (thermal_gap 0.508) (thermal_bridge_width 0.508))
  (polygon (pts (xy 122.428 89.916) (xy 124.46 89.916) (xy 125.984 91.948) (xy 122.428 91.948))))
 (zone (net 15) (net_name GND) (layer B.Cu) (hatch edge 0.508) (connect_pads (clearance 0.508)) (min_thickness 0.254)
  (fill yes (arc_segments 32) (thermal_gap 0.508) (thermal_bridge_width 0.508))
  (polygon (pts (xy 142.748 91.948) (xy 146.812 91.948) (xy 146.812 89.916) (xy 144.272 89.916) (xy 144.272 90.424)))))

